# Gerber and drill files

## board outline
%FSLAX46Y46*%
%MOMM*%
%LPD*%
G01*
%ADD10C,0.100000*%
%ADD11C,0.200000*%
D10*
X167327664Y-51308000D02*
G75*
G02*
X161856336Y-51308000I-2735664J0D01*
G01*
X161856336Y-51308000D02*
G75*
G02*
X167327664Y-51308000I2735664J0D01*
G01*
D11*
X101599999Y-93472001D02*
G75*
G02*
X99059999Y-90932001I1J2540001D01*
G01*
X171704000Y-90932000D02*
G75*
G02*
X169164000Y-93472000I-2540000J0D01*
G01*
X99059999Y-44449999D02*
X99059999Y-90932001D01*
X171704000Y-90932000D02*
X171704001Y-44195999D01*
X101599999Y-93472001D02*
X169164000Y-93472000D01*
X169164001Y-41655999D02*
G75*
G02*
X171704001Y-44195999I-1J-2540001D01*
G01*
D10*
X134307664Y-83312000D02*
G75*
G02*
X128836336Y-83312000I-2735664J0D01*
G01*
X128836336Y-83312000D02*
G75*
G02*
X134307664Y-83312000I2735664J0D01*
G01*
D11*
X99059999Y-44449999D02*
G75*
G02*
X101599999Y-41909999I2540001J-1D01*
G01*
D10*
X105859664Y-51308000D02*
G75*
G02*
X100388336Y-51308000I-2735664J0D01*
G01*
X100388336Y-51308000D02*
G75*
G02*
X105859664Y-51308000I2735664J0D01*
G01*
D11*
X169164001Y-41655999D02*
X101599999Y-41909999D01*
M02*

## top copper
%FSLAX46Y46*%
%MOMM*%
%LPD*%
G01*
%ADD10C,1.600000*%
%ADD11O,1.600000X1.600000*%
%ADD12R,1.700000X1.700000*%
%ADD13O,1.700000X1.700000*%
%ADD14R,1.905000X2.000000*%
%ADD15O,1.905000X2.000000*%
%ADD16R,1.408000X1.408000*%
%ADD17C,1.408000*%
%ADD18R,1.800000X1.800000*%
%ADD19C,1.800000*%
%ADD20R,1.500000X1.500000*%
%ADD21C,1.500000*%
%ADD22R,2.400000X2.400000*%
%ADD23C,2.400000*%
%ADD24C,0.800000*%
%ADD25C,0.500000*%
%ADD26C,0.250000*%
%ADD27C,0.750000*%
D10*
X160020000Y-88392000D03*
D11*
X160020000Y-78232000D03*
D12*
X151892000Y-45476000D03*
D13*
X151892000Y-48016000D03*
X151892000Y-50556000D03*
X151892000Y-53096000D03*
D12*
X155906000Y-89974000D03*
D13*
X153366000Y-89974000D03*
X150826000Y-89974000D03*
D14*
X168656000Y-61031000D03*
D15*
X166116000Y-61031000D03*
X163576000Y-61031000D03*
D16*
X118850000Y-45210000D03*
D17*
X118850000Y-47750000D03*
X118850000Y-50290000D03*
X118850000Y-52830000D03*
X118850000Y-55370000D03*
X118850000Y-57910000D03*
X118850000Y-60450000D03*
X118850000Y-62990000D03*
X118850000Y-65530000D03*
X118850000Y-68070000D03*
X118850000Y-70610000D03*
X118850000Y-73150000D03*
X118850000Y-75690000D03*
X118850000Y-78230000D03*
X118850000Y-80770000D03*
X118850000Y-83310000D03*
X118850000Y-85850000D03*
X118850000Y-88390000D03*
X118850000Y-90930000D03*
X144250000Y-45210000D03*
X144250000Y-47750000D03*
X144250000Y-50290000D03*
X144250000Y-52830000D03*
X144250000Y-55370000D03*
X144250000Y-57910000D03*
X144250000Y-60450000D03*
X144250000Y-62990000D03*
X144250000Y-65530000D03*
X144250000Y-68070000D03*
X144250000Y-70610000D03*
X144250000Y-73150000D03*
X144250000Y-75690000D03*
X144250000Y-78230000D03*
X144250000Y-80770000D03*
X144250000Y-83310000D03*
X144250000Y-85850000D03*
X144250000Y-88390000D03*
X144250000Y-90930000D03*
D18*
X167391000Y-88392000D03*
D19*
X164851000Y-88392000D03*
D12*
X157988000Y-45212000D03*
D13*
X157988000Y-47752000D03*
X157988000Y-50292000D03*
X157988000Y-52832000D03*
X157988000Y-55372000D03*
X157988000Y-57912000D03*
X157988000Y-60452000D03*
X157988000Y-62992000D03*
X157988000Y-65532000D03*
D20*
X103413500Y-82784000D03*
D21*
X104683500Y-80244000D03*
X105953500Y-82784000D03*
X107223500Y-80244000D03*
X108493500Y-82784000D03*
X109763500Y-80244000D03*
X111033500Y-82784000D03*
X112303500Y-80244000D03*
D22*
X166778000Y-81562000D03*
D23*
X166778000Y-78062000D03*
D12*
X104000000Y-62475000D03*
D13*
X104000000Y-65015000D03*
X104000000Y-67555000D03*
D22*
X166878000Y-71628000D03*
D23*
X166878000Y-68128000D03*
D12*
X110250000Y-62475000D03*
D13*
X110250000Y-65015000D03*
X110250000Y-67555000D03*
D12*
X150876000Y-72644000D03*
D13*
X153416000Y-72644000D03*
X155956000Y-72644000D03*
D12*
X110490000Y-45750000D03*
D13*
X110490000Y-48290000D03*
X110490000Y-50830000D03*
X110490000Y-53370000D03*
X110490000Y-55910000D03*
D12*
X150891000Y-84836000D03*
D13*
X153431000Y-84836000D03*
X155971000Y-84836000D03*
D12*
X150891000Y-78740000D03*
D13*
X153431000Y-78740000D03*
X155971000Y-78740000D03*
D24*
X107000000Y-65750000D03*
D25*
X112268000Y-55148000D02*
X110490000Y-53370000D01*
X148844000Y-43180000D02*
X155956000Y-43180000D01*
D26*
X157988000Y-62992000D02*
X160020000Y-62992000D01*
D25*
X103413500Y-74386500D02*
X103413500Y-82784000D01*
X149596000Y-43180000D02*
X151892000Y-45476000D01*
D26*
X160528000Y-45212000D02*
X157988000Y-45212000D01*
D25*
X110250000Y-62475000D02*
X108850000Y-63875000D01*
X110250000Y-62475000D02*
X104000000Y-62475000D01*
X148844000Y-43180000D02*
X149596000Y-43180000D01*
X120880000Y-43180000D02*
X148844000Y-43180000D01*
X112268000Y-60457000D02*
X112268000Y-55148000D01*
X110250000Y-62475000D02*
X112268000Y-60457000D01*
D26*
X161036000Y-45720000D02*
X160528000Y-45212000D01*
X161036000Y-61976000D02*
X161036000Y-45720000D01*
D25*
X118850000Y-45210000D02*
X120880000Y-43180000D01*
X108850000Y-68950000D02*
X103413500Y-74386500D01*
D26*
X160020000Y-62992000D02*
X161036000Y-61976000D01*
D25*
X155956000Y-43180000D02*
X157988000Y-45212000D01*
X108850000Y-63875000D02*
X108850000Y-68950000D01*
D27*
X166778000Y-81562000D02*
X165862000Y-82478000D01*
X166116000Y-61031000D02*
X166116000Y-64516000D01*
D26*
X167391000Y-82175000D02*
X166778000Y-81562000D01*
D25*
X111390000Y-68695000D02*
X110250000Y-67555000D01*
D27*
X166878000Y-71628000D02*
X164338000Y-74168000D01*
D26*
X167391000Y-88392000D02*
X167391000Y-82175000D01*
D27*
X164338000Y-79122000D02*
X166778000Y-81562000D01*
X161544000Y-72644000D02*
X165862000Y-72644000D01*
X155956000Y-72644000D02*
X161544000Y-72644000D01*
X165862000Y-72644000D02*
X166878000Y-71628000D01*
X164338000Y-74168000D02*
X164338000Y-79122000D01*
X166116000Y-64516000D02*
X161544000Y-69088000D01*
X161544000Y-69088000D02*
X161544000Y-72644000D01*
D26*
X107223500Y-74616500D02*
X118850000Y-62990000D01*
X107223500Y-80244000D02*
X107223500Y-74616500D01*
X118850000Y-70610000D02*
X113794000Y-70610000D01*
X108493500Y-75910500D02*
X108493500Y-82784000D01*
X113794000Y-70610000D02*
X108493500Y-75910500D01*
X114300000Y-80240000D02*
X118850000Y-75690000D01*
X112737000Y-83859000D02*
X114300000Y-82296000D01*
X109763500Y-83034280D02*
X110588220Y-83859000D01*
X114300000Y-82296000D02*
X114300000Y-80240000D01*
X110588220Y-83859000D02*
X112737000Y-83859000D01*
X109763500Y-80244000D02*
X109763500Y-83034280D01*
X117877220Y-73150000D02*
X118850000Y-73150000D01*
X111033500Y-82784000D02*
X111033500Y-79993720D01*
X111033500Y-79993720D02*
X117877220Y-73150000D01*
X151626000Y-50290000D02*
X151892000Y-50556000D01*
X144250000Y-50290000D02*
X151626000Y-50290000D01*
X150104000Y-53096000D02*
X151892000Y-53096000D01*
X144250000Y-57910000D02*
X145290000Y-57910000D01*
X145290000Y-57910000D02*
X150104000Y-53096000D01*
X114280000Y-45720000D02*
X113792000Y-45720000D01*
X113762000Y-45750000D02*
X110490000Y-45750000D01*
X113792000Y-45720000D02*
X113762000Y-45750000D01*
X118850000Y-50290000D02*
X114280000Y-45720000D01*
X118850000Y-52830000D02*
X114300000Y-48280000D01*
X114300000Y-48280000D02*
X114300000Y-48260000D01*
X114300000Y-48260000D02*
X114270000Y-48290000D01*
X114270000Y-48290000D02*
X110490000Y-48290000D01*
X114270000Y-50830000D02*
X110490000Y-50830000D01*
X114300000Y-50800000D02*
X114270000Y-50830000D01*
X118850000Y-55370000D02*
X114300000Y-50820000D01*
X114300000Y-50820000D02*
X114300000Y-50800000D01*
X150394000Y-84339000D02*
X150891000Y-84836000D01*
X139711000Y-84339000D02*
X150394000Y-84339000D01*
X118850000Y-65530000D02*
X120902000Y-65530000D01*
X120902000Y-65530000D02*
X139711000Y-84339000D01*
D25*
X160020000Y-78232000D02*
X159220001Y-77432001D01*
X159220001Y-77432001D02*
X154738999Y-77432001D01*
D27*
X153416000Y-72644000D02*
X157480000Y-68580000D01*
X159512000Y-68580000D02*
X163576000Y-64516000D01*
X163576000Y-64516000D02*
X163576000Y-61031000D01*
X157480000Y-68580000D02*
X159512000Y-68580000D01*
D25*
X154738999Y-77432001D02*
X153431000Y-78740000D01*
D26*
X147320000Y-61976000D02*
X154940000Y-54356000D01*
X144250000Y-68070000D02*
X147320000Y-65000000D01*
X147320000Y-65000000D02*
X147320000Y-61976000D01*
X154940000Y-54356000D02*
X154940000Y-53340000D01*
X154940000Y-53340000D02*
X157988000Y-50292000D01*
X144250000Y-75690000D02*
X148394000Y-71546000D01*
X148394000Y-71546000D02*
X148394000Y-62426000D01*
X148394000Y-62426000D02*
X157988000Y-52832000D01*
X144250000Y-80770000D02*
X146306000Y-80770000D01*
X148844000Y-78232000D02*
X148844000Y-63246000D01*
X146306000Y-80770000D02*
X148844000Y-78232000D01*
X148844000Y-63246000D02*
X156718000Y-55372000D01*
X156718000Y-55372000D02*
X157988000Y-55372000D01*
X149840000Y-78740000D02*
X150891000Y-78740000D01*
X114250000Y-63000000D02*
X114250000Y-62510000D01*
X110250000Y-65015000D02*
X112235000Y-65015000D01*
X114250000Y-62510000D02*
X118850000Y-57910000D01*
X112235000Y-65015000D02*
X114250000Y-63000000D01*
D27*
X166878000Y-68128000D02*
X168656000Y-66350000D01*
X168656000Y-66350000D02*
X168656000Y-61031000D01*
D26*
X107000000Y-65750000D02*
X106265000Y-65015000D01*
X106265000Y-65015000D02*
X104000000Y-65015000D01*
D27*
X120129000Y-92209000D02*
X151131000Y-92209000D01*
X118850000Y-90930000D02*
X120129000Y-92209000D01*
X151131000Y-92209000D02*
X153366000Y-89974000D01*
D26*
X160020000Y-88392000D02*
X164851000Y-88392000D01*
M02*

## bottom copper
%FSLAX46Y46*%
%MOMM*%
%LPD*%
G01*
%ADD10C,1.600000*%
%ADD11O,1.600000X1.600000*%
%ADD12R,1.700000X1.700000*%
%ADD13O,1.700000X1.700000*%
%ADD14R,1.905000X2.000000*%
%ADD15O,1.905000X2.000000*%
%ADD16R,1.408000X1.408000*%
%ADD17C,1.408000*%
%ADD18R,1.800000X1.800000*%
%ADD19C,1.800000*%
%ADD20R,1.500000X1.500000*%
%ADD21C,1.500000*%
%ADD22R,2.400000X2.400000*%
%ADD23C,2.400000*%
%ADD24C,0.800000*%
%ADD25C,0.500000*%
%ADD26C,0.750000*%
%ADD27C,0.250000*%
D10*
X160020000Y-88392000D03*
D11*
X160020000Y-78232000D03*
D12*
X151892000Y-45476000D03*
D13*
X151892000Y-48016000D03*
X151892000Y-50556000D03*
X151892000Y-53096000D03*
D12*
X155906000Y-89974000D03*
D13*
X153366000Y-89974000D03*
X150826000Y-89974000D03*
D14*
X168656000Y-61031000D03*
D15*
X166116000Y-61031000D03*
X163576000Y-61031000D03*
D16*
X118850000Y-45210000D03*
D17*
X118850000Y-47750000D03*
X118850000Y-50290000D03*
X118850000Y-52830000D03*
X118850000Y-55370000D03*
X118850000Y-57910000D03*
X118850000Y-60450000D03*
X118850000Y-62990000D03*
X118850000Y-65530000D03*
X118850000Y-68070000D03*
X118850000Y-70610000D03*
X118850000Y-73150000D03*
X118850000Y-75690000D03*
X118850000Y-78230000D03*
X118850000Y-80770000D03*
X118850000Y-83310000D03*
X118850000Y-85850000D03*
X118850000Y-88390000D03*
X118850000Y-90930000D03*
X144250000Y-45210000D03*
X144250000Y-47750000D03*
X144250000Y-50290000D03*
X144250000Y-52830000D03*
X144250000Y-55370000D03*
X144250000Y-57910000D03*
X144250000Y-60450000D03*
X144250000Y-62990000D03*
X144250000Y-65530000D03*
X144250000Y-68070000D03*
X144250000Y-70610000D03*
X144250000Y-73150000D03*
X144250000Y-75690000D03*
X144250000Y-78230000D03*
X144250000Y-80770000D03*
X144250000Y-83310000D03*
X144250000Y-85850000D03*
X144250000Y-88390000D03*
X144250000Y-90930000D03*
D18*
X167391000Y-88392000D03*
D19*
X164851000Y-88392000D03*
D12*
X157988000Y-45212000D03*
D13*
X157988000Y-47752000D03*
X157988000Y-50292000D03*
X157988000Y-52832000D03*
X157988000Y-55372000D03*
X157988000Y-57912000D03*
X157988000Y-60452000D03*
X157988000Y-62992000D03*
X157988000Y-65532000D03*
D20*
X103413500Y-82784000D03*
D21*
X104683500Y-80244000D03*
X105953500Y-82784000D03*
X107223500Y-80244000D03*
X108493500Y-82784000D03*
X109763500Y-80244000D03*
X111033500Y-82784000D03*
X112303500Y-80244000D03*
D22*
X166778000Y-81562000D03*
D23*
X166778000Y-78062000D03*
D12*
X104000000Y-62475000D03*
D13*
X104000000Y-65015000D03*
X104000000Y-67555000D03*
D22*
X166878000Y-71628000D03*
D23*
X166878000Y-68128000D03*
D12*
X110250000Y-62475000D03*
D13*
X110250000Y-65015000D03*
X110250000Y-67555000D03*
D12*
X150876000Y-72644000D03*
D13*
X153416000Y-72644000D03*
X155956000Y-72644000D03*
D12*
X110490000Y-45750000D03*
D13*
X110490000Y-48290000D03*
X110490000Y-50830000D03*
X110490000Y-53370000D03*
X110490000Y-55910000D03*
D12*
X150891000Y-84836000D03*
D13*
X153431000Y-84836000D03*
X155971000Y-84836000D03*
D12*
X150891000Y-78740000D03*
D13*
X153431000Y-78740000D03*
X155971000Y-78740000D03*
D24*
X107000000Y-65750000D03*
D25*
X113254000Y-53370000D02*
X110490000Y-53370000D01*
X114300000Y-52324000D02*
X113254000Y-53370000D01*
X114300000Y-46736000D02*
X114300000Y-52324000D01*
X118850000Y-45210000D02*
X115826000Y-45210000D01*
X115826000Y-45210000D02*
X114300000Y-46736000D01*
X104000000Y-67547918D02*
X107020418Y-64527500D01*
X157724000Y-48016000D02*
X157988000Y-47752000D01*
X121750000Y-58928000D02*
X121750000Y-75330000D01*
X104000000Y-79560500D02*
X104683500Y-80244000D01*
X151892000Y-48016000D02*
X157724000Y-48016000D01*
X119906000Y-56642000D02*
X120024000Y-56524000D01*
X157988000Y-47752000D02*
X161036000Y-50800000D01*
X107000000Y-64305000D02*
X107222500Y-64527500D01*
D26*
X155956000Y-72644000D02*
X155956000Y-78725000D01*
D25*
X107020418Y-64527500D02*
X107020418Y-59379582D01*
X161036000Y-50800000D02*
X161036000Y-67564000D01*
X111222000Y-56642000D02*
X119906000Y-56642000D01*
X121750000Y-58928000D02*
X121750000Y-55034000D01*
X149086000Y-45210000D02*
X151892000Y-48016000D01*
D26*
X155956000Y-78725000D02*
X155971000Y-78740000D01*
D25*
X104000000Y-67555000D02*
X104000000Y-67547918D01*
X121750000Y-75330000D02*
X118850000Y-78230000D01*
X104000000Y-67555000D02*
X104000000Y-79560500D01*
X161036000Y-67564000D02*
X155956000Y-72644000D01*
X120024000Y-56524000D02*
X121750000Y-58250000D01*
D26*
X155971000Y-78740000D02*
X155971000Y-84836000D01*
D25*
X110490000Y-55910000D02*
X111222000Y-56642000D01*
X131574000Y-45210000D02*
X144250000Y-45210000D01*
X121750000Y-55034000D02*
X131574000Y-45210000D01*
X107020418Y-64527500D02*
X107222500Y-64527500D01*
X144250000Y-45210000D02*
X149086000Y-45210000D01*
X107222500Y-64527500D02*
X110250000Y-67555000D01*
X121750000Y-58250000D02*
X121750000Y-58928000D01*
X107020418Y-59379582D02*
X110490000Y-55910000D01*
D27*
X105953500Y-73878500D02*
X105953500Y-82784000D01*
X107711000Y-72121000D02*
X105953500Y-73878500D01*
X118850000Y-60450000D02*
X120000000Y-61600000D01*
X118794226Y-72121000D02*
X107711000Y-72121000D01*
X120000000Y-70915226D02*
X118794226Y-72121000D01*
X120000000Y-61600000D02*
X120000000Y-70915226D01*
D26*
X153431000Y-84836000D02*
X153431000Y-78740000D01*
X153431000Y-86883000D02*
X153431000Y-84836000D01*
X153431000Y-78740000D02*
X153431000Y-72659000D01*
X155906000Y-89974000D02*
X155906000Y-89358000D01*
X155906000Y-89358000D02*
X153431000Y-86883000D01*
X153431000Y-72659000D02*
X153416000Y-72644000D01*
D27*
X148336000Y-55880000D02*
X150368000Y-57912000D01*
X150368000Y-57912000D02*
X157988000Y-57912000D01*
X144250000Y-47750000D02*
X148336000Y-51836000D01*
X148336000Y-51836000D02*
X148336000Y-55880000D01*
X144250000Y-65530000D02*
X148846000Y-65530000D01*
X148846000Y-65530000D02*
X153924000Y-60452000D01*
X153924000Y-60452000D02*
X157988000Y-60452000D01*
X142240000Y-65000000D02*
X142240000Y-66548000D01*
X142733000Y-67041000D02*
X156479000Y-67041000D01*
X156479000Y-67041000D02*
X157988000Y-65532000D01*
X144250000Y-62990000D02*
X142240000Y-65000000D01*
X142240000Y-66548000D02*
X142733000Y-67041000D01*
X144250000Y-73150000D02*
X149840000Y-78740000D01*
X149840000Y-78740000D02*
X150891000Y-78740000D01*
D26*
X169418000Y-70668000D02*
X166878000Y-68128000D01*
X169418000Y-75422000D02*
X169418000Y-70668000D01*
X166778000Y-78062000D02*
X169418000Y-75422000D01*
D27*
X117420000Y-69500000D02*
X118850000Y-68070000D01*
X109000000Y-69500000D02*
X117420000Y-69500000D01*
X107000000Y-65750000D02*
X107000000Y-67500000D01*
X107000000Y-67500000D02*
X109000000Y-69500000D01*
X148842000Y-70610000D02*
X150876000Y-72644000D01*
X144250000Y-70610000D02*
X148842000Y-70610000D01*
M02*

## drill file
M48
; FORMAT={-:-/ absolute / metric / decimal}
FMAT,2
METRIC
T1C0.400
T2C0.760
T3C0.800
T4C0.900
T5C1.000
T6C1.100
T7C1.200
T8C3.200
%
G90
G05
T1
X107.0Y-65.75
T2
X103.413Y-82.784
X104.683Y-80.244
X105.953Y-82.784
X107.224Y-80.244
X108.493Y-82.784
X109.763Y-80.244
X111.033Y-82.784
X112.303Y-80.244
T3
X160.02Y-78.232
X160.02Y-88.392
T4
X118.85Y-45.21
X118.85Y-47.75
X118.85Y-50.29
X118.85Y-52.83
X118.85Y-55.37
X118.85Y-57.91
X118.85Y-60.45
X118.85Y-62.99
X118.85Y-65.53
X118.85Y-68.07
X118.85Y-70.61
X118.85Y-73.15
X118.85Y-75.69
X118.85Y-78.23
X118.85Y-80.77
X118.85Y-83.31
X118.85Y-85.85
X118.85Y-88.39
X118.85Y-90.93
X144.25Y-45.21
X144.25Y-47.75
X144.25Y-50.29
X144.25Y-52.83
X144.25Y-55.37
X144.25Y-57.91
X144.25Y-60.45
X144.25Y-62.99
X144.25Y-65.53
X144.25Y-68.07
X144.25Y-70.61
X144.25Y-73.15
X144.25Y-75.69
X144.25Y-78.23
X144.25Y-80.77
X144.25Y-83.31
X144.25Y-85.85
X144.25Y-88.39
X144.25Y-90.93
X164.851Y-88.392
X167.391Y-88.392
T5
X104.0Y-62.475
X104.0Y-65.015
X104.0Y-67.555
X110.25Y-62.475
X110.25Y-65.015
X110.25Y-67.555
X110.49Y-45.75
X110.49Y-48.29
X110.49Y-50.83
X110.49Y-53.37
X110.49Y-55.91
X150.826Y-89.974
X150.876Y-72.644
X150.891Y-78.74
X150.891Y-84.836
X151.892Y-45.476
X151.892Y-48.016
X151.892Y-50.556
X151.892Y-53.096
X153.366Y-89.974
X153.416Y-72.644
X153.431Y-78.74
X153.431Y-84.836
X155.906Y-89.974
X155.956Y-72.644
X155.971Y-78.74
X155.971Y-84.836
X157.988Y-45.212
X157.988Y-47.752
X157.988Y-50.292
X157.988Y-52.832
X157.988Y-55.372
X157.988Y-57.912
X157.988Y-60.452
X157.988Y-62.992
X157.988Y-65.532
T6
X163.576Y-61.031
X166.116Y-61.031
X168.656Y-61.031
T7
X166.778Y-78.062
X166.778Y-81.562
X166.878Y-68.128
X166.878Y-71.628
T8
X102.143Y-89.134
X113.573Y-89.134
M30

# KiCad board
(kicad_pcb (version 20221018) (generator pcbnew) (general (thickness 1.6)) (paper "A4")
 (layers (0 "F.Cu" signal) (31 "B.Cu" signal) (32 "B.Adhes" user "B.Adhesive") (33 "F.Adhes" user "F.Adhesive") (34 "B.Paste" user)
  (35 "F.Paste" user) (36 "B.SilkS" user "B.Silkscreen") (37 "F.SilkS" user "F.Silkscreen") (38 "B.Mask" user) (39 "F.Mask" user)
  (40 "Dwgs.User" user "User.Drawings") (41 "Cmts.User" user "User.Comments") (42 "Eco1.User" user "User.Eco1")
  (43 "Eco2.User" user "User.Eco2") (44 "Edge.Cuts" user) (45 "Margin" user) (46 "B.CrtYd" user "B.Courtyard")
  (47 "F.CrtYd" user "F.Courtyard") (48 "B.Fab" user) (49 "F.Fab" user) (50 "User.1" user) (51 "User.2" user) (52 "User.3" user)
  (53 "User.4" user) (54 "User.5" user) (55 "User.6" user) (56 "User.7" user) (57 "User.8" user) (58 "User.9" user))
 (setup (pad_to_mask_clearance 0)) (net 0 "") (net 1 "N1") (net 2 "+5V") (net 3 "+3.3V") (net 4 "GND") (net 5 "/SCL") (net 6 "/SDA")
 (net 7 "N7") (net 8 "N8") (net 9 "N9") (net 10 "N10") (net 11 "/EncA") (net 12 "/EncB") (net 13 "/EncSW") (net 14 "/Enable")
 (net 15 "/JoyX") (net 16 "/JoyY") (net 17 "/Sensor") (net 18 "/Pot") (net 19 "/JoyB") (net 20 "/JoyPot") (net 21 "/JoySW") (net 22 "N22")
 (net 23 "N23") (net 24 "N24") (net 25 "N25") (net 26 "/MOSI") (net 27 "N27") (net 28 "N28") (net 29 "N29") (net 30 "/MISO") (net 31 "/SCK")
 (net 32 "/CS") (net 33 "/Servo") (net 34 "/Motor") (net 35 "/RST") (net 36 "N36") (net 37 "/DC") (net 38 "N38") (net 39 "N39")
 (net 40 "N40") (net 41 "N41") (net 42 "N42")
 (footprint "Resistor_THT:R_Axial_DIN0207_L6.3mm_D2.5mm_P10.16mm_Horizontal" (layer "F.Cu") (at 160.02 88.392 90)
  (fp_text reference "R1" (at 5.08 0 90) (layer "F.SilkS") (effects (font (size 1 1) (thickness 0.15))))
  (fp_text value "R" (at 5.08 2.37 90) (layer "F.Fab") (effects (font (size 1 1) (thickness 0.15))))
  (pad "1" thru_hole circle (at 0 0 90) (size 1.6 1.6) (drill 0.8) (layers "*.Cu" "*.Mask") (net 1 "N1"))
  (pad "2" thru_hole oval (at 10.16 0 90) (size 1.6 1.6) (drill 0.8) (layers "*.Cu" "*.Mask") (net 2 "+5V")))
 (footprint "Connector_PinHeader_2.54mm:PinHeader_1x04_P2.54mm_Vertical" (layer "F.Cu") (at 151.892 45.476)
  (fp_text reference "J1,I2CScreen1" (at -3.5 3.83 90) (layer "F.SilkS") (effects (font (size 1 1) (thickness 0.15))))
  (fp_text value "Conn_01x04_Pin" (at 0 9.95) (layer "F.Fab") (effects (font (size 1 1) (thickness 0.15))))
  (pad "1" thru_hole rect (at 0 0) (size 1.7 1.7) (drill 1) (layers "*.Cu" "*.Mask") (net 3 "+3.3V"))
  (pad "2" thru_hole oval (at 0 2.54) (size 1.7 1.7) (drill 1) (layers "*.Cu" "*.Mask") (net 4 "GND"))
  (pad "3" thru_hole oval (at 0 5.08) (size 1.7 1.7) (drill 1) (layers "*.Cu" "*.Mask") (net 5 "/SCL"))
  (pad "4" thru_hole oval (at 0 7.62) (size 1.7 1.7) (drill 1) (layers "*.Cu" "*.Mask") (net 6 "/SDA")))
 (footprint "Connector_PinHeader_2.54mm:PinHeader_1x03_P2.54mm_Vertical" (layer "F.Cu") (at 155.906 89.974 -90)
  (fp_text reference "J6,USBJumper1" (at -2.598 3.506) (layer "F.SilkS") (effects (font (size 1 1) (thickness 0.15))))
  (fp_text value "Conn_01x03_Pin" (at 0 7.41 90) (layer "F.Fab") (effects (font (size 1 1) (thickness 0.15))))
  (pad "1" thru_hole rect (at 0 0 270) (size 1.7 1.7) (drill 1) (layers "*.Cu" "*.Mask") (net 2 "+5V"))
  (pad "2" thru_hole oval (at 0 2.54 270) (size 1.7 1.7) (drill 1) (layers "*.Cu" "*.Mask") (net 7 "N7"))
  (pad "3" thru_hole oval (at 0 5.08 270) (size 1.7 1.7) (drill 1) (layers "*.Cu" "*.Mask") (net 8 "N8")))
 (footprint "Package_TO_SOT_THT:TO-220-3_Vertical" (layer "F.Cu") (at 168.656 61.031 180)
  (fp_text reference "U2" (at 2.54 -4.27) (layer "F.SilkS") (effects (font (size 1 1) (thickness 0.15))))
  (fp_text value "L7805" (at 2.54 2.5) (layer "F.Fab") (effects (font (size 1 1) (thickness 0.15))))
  (pad "1" thru_hole rect (at 0 0 180) (size 1.905 2) (drill 1.1) (layers "*.Cu" "*.Mask") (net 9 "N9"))
  (pad "2" thru_hole oval (at 2.54 0 180) (size 1.905 2) (drill 1.1) (layers "*.Cu" "*.Mask") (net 4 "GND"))
  (pad "3" thru_hole oval (at 5.08 0 180) (size 1.905 2) (drill 1.1) (layers "*.Cu" "*.Mask") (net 2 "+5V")))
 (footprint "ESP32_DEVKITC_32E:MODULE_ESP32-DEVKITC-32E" (layer "F.Cu") (at 131.55 68.045)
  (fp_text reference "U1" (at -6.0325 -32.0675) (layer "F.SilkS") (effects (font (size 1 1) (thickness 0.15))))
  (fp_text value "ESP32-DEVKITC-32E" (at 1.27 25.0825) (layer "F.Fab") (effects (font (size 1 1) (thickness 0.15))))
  (pad "J2_1" thru_hole rect (at -12.7 -22.835) (size 1.408 1.408) (drill 0.9) (layers "*.Cu" "*.Mask") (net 3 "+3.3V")
   (solder_mask_margin 0.102))
  (pad "J2_2" thru_hole circle (at -12.7 -20.295) (size 1.408 1.408) (drill 0.9) (layers "*.Cu" "*.Mask") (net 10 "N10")
   (solder_mask_margin 0.102))
  (pad "J2_3" thru_hole circle (at -12.7 -17.755) (size 1.408 1.408) (drill 0.9) (layers "*.Cu" "*.Mask") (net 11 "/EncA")
   (solder_mask_margin 0.102))
  (pad "J2_4" thru_hole circle (at -12.7 -15.215) (size 1.408 1.408) (drill 0.9) (layers "*.Cu" "*.Mask") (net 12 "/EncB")
   (solder_mask_margin 0.102))
  (pad "J2_5" thru_hole circle (at -12.7 -12.675) (size 1.408 1.408) (drill 0.9) (layers "*.Cu" "*.Mask") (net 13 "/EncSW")
   (solder_mask_margin 0.102))
  (pad "J2_6" thru_hole circle (at -12.7 -10.135) (size 1.408 1.408) (drill 0.9) (layers "*.Cu" "*.Mask") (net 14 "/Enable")
   (solder_mask_margin 0.102))
  (pad "J2_7" thru_hole circle (at -12.7 -7.595) (size 1.408 1.408) (drill 0.9) (layers "*.Cu" "*.Mask") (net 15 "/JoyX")
   (solder_mask_margin 0.102))
  (pad "J2_8" thru_hole circle (at -12.7 -5.055) (size 1.408 1.408) (drill 0.9) (layers "*.Cu" "*.Mask") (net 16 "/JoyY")
   (solder_mask_margin 0.102))
  (pad "J2_9" thru_hole circle (at -12.7 -2.515) (size 1.408 1.408) (drill 0.9) (layers "*.Cu" "*.Mask") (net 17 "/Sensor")
   (solder_mask_margin 0.102))
  (pad "J2_10" thru_hole circle (at -12.7 0.025) (size 1.408 1.408) (drill 0.9) (layers "*.Cu" "*.Mask") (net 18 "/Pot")
   (solder_mask_margin 0.102))
  (pad "J2_11" thru_hole circle (at -12.7 2.565) (size 1.408 1.408) (drill 0.9) (layers "*.Cu" "*.Mask") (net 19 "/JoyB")
   (solder_mask_margin 0.102))
  (pad "J2_12" thru_hole circle (at -12.7 5.105) (size 1.408 1.408) (drill 0.9) (layers "*.Cu" "*.Mask") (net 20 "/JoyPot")
   (solder_mask_margin 0.102))
  (pad "J2_13" thru_hole circle (at -12.7 7.645) (size 1.408 1.408) (drill 0.9) (layers "*.Cu" "*.Mask") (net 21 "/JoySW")
   (solder_mask_margin 0.102))
  (pad "J2_14" thru_hole circle (at -12.7 10.185) (size 1.408 1.408) (drill 0.9) (layers "*.Cu" "*.Mask") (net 4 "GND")
   (solder_mask_margin 0.102))
  (pad "J2_15" thru_hole circle (at -12.7 12.725) (size 1.408 1.408) (drill 0.9) (layers "*.Cu" "*.Mask") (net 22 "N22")
   (solder_mask_margin 0.102))
  (pad "J2_16" thru_hole circle (at -12.7 15.265) (size 1.408 1.408) (drill 0.9) (layers "*.Cu" "*.Mask") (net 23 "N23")
   (solder_mask_margin 0.102))
  (pad "J2_17" thru_hole circle (at -12.7 17.805) (size 1.408 1.408) (drill 0.9) (layers "*.Cu" "*.Mask") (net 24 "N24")
   (solder_mask_margin 0.102))
  (pad "J2_18" thru_hole circle (at -12.7 20.345) (size 1.408 1.408) (drill 0.9) (layers "*.Cu" "*.Mask") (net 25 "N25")
   (solder_mask_margin 0.102))
  (pad "J2_19" thru_hole circle (at -12.7 22.885) (size 1.408 1.408) (drill 0.9) (layers "*.Cu" "*.Mask") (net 7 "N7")
   (solder_mask_margin 0.102))
  (pad "J3_1" thru_hole circle (at 12.7 -22.835) (size 1.408 1.408) (drill 0.9) (layers "*.Cu" "*.Mask") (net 4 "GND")
   (solder_mask_margin 0.102))
  (pad "J3_2" thru_hole circle (at 12.7 -20.295) (size 1.408 1.408) (drill 0.9) (layers "*.Cu" "*.Mask") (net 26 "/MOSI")
   (solder_mask_margin 0.102))
  (pad "J3_3" thru_hole circle (at 12.7 -17.755) (size 1.408 1.408) (drill 0.9) (layers "*.Cu" "*.Mask") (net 5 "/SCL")
   (solder_mask_margin 0.102))
  (pad "J3_4" thru_hole circle (at 12.7 -15.215) (size 1.408 1.408) (drill 0.9) (layers "*.Cu" "*.Mask") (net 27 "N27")
   (solder_mask_margin 0.102))
  (pad "J3_5" thru_hole circle (at 12.7 -12.675) (size 1.408 1.408) (drill 0.9) (layers "*.Cu" "*.Mask") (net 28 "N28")
   (solder_mask_margin 0.102))
  (pad "J3_6" thru_hole circle (at 12.7 -10.135) (size 1.408 1.408) (drill 0.9) (layers "*.Cu" "*.Mask") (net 6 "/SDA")
   (solder_mask_margin 0.102))
  (pad "J3_7" thru_hole circle (at 12.7 -7.595) (size 1.408 1.408) (drill 0.9) (layers "*.Cu" "*.Mask") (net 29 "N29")
   (solder_mask_margin 0.102))
  (pad "J3_8" thru_hole circle (at 12.7 -5.055) (size 1.408 1.408) (drill 0.9) (layers "*.Cu" "*.Mask") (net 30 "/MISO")
   (solder_mask_margin 0.102))
  (pad "J3_9" thru_hole circle (at 12.7 -2.515) (size 1.408 1.408) (drill 0.9) (layers "*.Cu" "*.Mask") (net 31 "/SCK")
   (solder_mask_margin 0.102))
  (pad "J3_10" thru_hole circle (at 12.7 0.025) (size 1.408 1.408) (drill 0.9) (layers "*.Cu" "*.Mask") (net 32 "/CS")
   (solder_mask_margin 0.102))
  (pad "J3_11" thru_hole circle (at 12.7 2.565) (size 1.408 1.408) (drill 0.9) (layers "*.Cu" "*.Mask") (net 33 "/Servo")
   (solder_mask_margin 0.102))
  (pad "J3_12" thru_hole circle (at 12.7 5.105) (size 1.408 1.408) (drill 0.9) (layers "*.Cu" "*.Mask") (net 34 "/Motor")
   (solder_mask_margin 0.102))
  (pad "J3_13" thru_hole circle (at 12.7 7.645) (size 1.408 1.408) (drill 0.9) (layers "*.Cu" "*.Mask") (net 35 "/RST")
   (solder_mask_margin 0.102))
  (pad "J3_14" thru_hole circle (at 12.7 10.185) (size 1.408 1.408) (drill 0.9) (layers "*.Cu" "*.Mask") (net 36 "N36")
   (solder_mask_margin 0.102))
  (pad "J3_15" thru_hole circle (at 12.7 12.725) (size 1.408 1.408) (drill 0.9) (layers "*.Cu" "*.Mask") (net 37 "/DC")
   (solder_mask_margin 0.102))
  (pad "J3_16" thru_hole circle (at 12.7 15.265) (size 1.408 1.408) (drill 0.9) (layers "*.Cu" "*.Mask") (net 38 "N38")
   (solder_mask_margin 0.102))
  (pad "J3_17" thru_hole circle (at 12.7 17.805) (size 1.408 1.408) (drill 0.9) (layers "*.Cu" "*.Mask") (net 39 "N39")
   (solder_mask_margin 0.102))
  (pad "J3_18" thru_hole circle (at 12.7 20.345) (size 1.408 1.408) (drill 0.9) (layers "*.Cu" "*.Mask") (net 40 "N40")
   (solder_mask_margin 0.102))
  (pad "J3_19" thru_hole circle (at 12.7 22.885) (size 1.408 1.408) (drill 0.9) (layers "*.Cu" "*.Mask") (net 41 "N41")
   (solder_mask_margin 0.102)))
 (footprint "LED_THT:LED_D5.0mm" (layer "F.Cu") (at 167.391 88.392 180)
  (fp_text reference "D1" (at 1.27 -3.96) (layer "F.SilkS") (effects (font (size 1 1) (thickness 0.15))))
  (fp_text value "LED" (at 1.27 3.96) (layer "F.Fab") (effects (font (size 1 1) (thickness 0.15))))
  (pad "1" thru_hole rect (at 0 0 180) (size 1.8 1.8) (drill 0.9) (layers "*.Cu" "*.Mask") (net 4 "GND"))
  (pad "2" thru_hole circle (at 2.54 0 180) (size 1.8 1.8) (drill 0.9) (layers "*.Cu" "*.Mask") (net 1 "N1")))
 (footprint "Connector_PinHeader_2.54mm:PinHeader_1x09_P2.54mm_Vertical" (layer "F.Cu") (at 157.988 45.212)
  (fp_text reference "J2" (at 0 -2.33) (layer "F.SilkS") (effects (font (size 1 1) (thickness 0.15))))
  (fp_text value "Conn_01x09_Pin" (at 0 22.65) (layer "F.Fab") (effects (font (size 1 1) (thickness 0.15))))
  (pad "1" thru_hole rect (at 0 0) (size 1.7 1.7) (drill 1) (layers "*.Cu" "*.Mask") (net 3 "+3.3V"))
  (pad "2" thru_hole oval (at 0 2.54) (size 1.7 1.7) (drill 1) (layers "*.Cu" "*.Mask") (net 4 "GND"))
  (pad "3" thru_hole oval (at 0 5.08) (size 1.7 1.7) (drill 1) (layers "*.Cu" "*.Mask") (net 32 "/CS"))
  (pad "4" thru_hole oval (at 0 7.62) (size 1.7 1.7) (drill 1) (layers "*.Cu" "*.Mask") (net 35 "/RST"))
  (pad "5" thru_hole oval (at 0 10.16) (size 1.7 1.7) (drill 1) (layers "*.Cu" "*.Mask") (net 37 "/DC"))
  (pad "6" thru_hole oval (at 0 12.7) (size 1.7 1.7) (drill 1) (layers "*.Cu" "*.Mask") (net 26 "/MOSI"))
  (pad "7" thru_hole oval (at 0 15.24) (size 1.7 1.7) (drill 1) (layers "*.Cu" "*.Mask") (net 31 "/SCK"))
  (pad "8" thru_hole oval (at 0 17.78) (size 1.7 1.7) (drill 1) (layers "*.Cu" "*.Mask") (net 3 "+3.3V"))
  (pad "9" thru_hole oval (at 0 20.32) (size 1.7 1.7) (drill 1) (layers "*.Cu" "*.Mask") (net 30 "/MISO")))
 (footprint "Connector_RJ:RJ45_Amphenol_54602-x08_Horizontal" (layer "F.Cu") (at 103.4135 82.784)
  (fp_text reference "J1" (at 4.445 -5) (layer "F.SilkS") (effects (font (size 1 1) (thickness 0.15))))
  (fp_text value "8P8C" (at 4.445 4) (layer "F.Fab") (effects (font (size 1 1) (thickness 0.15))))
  (pad "" np_thru_hole circle (at -1.27 6.35) (size 3.2 3.2) (drill 3.2) (layers "*.Cu" "*.Mask"))
  (pad "" np_thru_hole circle (at 10.16 6.35) (size 3.2 3.2) (drill 3.2) (layers "*.Cu" "*.Mask"))
  (pad "1" thru_hole rect (at 0 0) (size 1.5 1.5) (drill 0.76) (layers "*.Cu" "*.Mask") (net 3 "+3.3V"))
  (pad "2" thru_hole circle (at 1.27 -2.54) (size 1.5 1.5) (drill 0.76) (layers "*.Cu" "*.Mask") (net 4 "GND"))
  (pad "3" thru_hole circle (at 2.54 0) (size 1.5 1.5) (drill 0.76) (layers "*.Cu" "*.Mask") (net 15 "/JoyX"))
  (pad "4" thru_hole circle (at 3.81 -2.54) (size 1.5 1.5) (drill 0.76) (layers "*.Cu" "*.Mask") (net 16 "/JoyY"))
  (pad "5" thru_hole circle (at 5.08 0) (size 1.5 1.5) (drill 0.76) (layers "*.Cu" "*.Mask") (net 19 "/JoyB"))
  (pad "6" thru_hole circle (at 6.35 -2.54) (size 1.5 1.5) (drill 0.76) (layers "*.Cu" "*.Mask") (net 21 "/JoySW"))
  (pad "7" thru_hole circle (at 7.62 0) (size 1.5 1.5) (drill 0.76) (layers "*.Cu" "*.Mask") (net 20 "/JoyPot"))
  (pad "8" thru_hole circle (at 8.89 -2.54) (size 1.5 1.5) (drill 0.76) (layers "*.Cu" "*.Mask") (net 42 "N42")))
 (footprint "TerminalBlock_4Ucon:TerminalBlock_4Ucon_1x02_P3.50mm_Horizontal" (layer "F.Cu") (at 166.778 81.562 90)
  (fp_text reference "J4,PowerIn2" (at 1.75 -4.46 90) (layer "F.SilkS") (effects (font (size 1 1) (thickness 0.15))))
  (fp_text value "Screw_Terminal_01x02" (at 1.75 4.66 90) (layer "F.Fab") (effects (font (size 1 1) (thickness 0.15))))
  (pad "1" thru_hole rect (at 0 0 90) (size 2.4 2.4) (drill 1.2) (layers "*.Cu" "*.Mask") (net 4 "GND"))
  (pad "2" thru_hole circle (at 3.5 0 90) (size 2.4 2.4) (drill 1.2) (layers "*.Cu" "*.Mask") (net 9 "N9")))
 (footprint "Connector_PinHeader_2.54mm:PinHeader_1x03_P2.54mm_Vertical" (layer "F.Cu") (at 104 62.475)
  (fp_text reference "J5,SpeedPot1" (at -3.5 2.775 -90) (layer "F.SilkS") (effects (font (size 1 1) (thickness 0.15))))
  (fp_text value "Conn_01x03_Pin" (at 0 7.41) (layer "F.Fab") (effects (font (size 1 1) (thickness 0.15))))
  (pad "1" thru_hole rect (at 0 0) (size 1.7 1.7) (drill 1) (layers "*.Cu" "*.Mask") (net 3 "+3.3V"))
  (pad "2" thru_hole oval (at 0 2.54) (size 1.7 1.7) (drill 1) (layers "*.Cu" "*.Mask") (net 18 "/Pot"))
  (pad "3" thru_hole oval (at 0 5.08) (size 1.7 1.7) (drill 1) (layers "*.Cu" "*.Mask") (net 4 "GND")))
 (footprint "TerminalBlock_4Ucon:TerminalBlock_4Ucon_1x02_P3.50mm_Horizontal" (layer "F.Cu") (at 166.878 71.628 90)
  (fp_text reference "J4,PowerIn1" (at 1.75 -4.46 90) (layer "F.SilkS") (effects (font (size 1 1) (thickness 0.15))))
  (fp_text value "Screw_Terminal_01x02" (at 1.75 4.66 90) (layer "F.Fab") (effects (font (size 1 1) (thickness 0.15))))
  (pad "1" thru_hole rect (at 0 0 90) (size 2.4 2.4) (drill 1.2) (layers "*.Cu" "*.Mask") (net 4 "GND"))
  (pad "2" thru_hole circle (at 3.5 0 90) (size 2.4 2.4) (drill 1.2) (layers "*.Cu" "*.Mask") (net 9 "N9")))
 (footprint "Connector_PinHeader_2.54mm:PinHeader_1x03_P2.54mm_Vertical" (layer "F.Cu") (at 110.25 62.475)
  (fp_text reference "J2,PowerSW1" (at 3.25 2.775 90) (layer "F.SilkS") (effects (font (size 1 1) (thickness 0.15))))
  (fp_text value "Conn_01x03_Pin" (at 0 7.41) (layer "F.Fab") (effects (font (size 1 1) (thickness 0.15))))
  (pad "1" thru_hole rect (at 0 0) (size 1.7 1.7) (drill 1) (layers "*.Cu" "*.Mask") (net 3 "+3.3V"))
  (pad "2" thru_hole oval (at 0 2.54) (size 1.7 1.7) (drill 1) (layers "*.Cu" "*.Mask") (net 14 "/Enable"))
  (pad "3" thru_hole oval (at 0 5.08) (size 1.7 1.7) (drill 1) (layers "*.Cu" "*.Mask") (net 4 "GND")))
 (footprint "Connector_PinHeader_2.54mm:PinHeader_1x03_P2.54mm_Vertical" (layer "F.Cu") (at 150.876 72.644 90)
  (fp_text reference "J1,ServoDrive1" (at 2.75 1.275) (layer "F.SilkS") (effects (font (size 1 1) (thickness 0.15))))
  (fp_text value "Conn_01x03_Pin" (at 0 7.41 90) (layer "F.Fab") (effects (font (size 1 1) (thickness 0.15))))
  (pad "1" thru_hole rect (at 0 0 90) (size 1.7 1.7) (drill 1) (layers "*.Cu" "*.Mask") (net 33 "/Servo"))
  (pad "2" thru_hole oval (at 0 2.54 90) (size 1.7 1.7) (drill 1) (layers "*.Cu" "*.Mask") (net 2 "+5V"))
  (pad "3" thru_hole oval (at 0 5.08 90) (size 1.7 1.7) (drill 1) (layers "*.Cu" "*.Mask") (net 4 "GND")))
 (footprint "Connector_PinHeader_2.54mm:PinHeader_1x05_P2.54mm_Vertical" (layer "F.Cu") (at 110.49 45.75)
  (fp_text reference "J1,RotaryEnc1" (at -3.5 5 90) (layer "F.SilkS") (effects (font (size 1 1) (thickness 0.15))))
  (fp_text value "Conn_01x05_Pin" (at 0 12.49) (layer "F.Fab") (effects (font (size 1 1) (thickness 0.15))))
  (pad "1" thru_hole rect (at 0 0) (size 1.7 1.7) (drill 1) (layers "*.Cu" "*.Mask") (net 11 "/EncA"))
  (pad "2" thru_hole oval (at 0 2.54) (size 1.7 1.7) (drill 1) (layers "*.Cu" "*.Mask") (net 12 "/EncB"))
  (pad "3" thru_hole oval (at 0 5.08) (size 1.7 1.7) (drill 1) (layers "*.Cu" "*.Mask") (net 13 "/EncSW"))
  (pad "4" thru_hole oval (at 0 7.62) (size 1.7 1.7) (drill 1) (layers "*.Cu" "*.Mask") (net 3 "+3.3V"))
  (pad "5" thru_hole oval (at 0 10.16) (size 1.7 1.7) (drill 1) (layers "*.Cu" "*.Mask") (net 4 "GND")))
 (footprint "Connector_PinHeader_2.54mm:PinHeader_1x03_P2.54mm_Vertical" (layer "F.Cu") (at 150.891 84.836 90)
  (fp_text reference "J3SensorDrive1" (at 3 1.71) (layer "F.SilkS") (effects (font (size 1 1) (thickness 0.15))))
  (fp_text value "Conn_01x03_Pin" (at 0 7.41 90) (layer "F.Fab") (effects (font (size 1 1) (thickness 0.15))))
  (pad "1" thru_hole rect (at 0 0 90) (size 1.7 1.7) (drill 1) (layers "*.Cu" "*.Mask") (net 17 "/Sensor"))
  (pad "2" thru_hole oval (at 0 2.54 90) (size 1.7 1.7) (drill 1) (layers "*.Cu" "*.Mask") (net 2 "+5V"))
  (pad "3" thru_hole oval (at 0 5.08 90) (size 1.7 1.7) (drill 1) (layers "*.Cu" "*.Mask") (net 4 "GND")))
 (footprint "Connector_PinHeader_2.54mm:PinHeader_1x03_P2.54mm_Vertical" (layer "F.Cu") (at 150.891 78.74 90)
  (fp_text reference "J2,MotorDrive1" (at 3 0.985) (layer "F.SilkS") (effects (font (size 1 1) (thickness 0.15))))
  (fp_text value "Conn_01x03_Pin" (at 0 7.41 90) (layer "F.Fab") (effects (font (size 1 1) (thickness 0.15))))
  (pad "1" thru_hole rect (at 0 0 90) (size 1.7 1.7) (drill 1) (layers "*.Cu" "*.Mask") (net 34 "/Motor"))
  (pad "2" thru_hole oval (at 0 2.54 90) (size 1.7 1.7) (drill 1) (layers "*.Cu" "*.Mask") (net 2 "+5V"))
  (pad "3" thru_hole oval (at 0 5.08 90) (size 1.7 1.7) (drill 1) (layers "*.Cu" "*.Mask") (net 4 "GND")))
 (gr_circle (center 164.592 51.308) (end 165.608 53.848) (stroke (width 0.1) (type default)) (fill none) (layer "Edge.Cuts"))
 (gr_arc (start 101.599999 93.472001) (mid 99.803948 92.728052) (end 99.059999 90.932001) (stroke (width 0.2) (type default))
  (layer "Edge.Cuts"))
 (gr_arc (start 171.704 90.932) (mid 170.960051 92.728051) (end 169.164 93.472) (stroke (width 0.2) (type default)) (layer "Edge.Cuts"))
 (gr_line (start 99.059999 44.449999) (end 99.059999 90.932001) (stroke (width 0.2) (type default)) (layer "Edge.Cuts"))
 (gr_line (start 171.704 90.932) (end 171.704001 44.195999) (stroke (width 0.2) (type default)) (layer "Edge.Cuts"))
 (gr_line (start 101.599999 93.472001) (end 169.164 93.472) (stroke (width 0.2) (type default)) (layer "Edge.Cuts"))
 (gr_arc (start 169.164001 41.655999) (mid 170.960052 42.399948) (end 171.704001 44.195999) (stroke (width 0.2) (type default))
  (layer "Edge.Cuts"))
 (gr_circle (center 131.572 83.312) (end 132.588 85.852) (stroke (width 0.1) (type default)) (fill none) (layer "Edge.Cuts"))
 (gr_arc (start 99.059999 44.449999) (mid 99.803948 42.653948) (end 101.599999 41.909999) (stroke (width 0.2) (type default))
  (layer "Edge.Cuts"))
 (gr_circle (center 103.124 51.308) (end 104.14 53.848) (stroke (width 0.1) (type default)) (fill none) (layer "Edge.Cuts"))
 (gr_line (start 169.164001 41.655999) (end 101.599999 41.909999) (stroke (width 0.2) (type default)) (layer "Edge.Cuts"))
 (segment (start 112.268 55.148) (end 110.49 53.37) (width 0.5) (layer "F.Cu") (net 3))
 (segment (start 148.844 43.18) (end 155.956 43.18) (width 0.5) (layer "F.Cu") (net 3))
 (segment (start 157.988 62.992) (end 160.02 62.992) (width 0.25) (layer "F.Cu") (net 3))
 (segment (start 103.4135 74.3865) (end 103.4135 82.784) (width 0.5) (layer "F.Cu") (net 3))
 (segment (start 149.596 43.18) (end 151.892 45.476) (width 0.5) (layer "F.Cu") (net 3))
 (segment (start 160.528 45.212) (end 157.988 45.212) (width 0.25) (layer "F.Cu") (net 3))
 (segment (start 110.25 62.475) (end 108.85 63.875) (width 0.5) (layer "F.Cu") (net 3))
 (segment (start 110.25 62.475) (end 104 62.475) (width 0.5) (layer "F.Cu") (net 3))
 (segment (start 148.844 43.18) (end 149.596 43.18) (width 0.5) (layer "F.Cu") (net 3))
 (segment (start 120.88 43.18) (end 148.844 43.18) (width 0.5) (layer "F.Cu") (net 3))
 (segment (start 112.268 60.457) (end 112.268 55.148) (width 0.5) (layer "F.Cu") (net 3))
 (segment (start 110.25 62.475) (end 112.268 60.457) (width 0.5) (layer "F.Cu") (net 3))
 (segment (start 161.036 45.72) (end 160.528 45.212) (width 0.25) (layer "F.Cu") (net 3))
 (segment (start 161.036 61.976) (end 161.036 45.72) (width 0.25) (layer "F.Cu") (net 3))
 (segment (start 118.85 45.21) (end 120.88 43.18) (width 0.5) (layer "F.Cu") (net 3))
 (segment (start 108.85 68.95) (end 103.4135 74.3865) (width 0.5) (layer "F.Cu") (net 3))
 (segment (start 160.02 62.992) (end 161.036 61.976) (width 0.25) (layer "F.Cu") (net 3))
 (segment (start 155.956 43.18) (end 157.988 45.212) (width 0.5) (layer "F.Cu") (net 3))
 (segment (start 108.85 63.875) (end 108.85 68.95) (width 0.5) (layer "F.Cu") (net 3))
 (segment (start 113.254 53.37) (end 110.49 53.37) (width 0.5) (layer "B.Cu") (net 3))
 (segment (start 114.3 52.324) (end 113.254 53.37) (width 0.5) (layer "B.Cu") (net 3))
 (segment (start 114.3 46.736) (end 114.3 52.324) (width 0.5) (layer "B.Cu") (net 3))
 (segment (start 118.85 45.21) (end 115.826 45.21) (width 0.5) (layer "B.Cu") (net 3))
 (segment (start 115.826 45.21) (end 114.3 46.736) (width 0.5) (layer "B.Cu") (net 3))
 (segment (start 166.778 81.562) (end 165.862 82.478) (width 0.75) (layer "F.Cu") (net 4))
 (segment (start 166.116 61.031) (end 166.116 64.516) (width 0.75) (layer "F.Cu") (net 4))
 (segment (start 167.391 82.175) (end 166.778 81.562) (width 0.25) (layer "F.Cu") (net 4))
 (segment (start 111.39 68.695) (end 110.25 67.555) (width 0.5) (layer "F.Cu") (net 4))
 (segment (start 166.878 71.628) (end 164.338 74.168) (width 0.75) (layer "F.Cu") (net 4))
 (segment (start 167.391 88.392) (end 167.391 82.175) (width 0.25) (layer "F.Cu") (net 4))
 (segment (start 164.338 79.122) (end 166.778 81.562) (width 0.75) (layer "F.Cu") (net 4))
 (segment (start 161.544 72.644) (end 165.862 72.644) (width 0.75) (layer "F.Cu") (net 4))
 (segment (start 155.956 72.644) (end 161.544 72.644) (width 0.75) (layer "F.Cu") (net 4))
 (segment (start 165.862 72.644) (end 166.878 71.628) (width 0.75) (layer "F.Cu") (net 4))
 (segment (start 164.338 74.168) (end 164.338 79.122) (width 0.75) (layer "F.Cu") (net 4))
 (segment (start 166.116 64.516) (end 161.544 69.088) (width 0.75) (layer "F.Cu") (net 4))
 (segment (start 161.544 69.088) (end 161.544 72.644) (width 0.75) (layer "F.Cu") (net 4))
 (segment (start 104 67.547918) (end 107.020418 64.5275) (width 0.5) (layer "B.Cu") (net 4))
 (segment (start 157.724 48.016) (end 157.988 47.752) (width 0.5) (layer "B.Cu") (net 4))
 (segment (start 121.75 58.928) (end 121.75 75.33) (width 0.5) (layer "B.Cu") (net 4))
 (segment (start 104 79.5605) (end 104.6835 80.244) (width 0.5) (layer "B.Cu") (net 4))
 (segment (start 151.892 48.016) (end 157.724 48.016) (width 0.5) (layer "B.Cu") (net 4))
 (segment (start 119.906 56.642) (end 120.024 56.524) (width 0.5) (layer "B.Cu") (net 4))
 (segment (start 157.988 47.752) (end 161.036 50.8) (width 0.5) (layer "B.Cu") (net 4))
 (segment (start 107 64.305) (end 107.2225 64.5275) (width 0.5) (layer "B.Cu") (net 4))
 (segment (start 155.956 72.644) (end 155.956 78.725) (width 0.75) (layer "B.Cu") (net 4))
 (segment (start 107.020418 64.5275) (end 107.020418 59.379582) (width 0.5) (layer "B.Cu") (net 4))
 (segment (start 161.036 50.8) (end 161.036 67.564) (width 0.5) (layer "B.Cu") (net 4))
 (segment (start 111.222 56.642) (end 119.906 56.642) (width 0.5) (layer "B.Cu") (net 4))
 (segment (start 121.75 58.928) (end 121.75 55.034) (width 0.5) (layer "B.Cu") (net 4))
 (segment (start 149.086 45.21) (end 151.892 48.016) (width 0.5) (layer "B.Cu") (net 4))
 (segment (start 155.956 78.725) (end 155.971 78.74) (width 0.75) (layer "B.Cu") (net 4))
 (segment (start 104 67.555) (end 104 67.547918) (width 0.5) (layer "B.Cu") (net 4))
 (segment (start 121.75 75.33) (end 118.85 78.23) (width 0.5) (layer "B.Cu") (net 4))
 (segment (start 104 67.555) (end 104 79.5605) (width 0.5) (layer "B.Cu") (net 4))
 (segment (start 161.036 67.564) (end 155.956 72.644) (width 0.5) (layer "B.Cu") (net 4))
 (segment (start 120.024 56.524) (end 121.75 58.25) (width 0.5) (layer "B.Cu") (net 4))
 (segment (start 155.971 78.74) (end 155.971 84.836) (width 0.75) (layer "B.Cu") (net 4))
 (segment (start 110.49 55.91) (end 111.222 56.642) (width 0.5) (layer "B.Cu") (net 4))
 (segment (start 131.574 45.21) (end 144.25 45.21) (width 0.5) (layer "B.Cu") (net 4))
 (segment (start 121.75 55.034) (end 131.574 45.21) (width 0.5) (layer "B.Cu") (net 4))
 (segment (start 107.020418 64.5275) (end 107.2225 64.5275) (width 0.5) (layer "B.Cu") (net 4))
 (segment (start 144.25 45.21) (end 149.086 45.21) (width 0.5) (layer "B.Cu") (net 4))
 (segment (start 107.2225 64.5275) (end 110.25 67.555) (width 0.5) (layer "B.Cu") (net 4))
 (segment (start 121.75 58.25) (end 121.75 58.928) (width 0.5) (layer "B.Cu") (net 4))
 (segment (start 107.020418 59.379582) (end 110.49 55.91) (width 0.5) (layer "B.Cu") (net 4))
 (segment (start 105.9535 73.8785) (end 105.9535 82.784) (width 0.25) (layer "B.Cu") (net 15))
 (segment (start 107.711 72.121) (end 105.9535 73.8785) (width 0.25) (layer "B.Cu") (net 15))
 (segment (start 118.85 60.45) (end 120 61.6) (width 0.25) (layer "B.Cu") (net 15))
 (segment (start 118.794226 72.121) (end 107.711 72.121) (width 0.25) (layer "B.Cu") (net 15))
 (segment (start 120 70.915226) (end 118.794226 72.121) (width 0.25) (layer "B.Cu") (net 15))
 (segment (start 120 61.6) (end 120 70.915226) (width 0.25) (layer "B.Cu") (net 15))
 (segment (start 107.2235 74.6165) (end 118.85 62.99) (width 0.25) (layer "F.Cu") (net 16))
 (segment (start 107.2235 80.244) (end 107.2235 74.6165) (width 0.25) (layer "F.Cu") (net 16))
 (segment (start 118.85 70.61) (end 113.794 70.61) (width 0.25) (layer "F.Cu") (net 19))
 (segment (start 108.4935 75.9105) (end 108.4935 82.784) (width 0.25) (layer "F.Cu") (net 19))
 (segment (start 113.794 70.61) (end 108.4935 75.9105) (width 0.25) (layer "F.Cu") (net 19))
 (segment (start 114.3 80.24) (end 118.85 75.69) (width 0.25) (layer "F.Cu") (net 21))
 (segment (start 112.737 83.859) (end 114.3 82.296) (width 0.25) (layer "F.Cu") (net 21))
 (segment (start 109.7635 83.03428) (end 110.58822 83.859) (width 0.25) (layer "F.Cu") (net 21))
 (segment (start 114.3 82.296) (end 114.3 80.24) (width 0.25) (layer "F.Cu") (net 21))
 (segment (start 110.58822 83.859) (end 112.737 83.859) (width 0.25) (layer "F.Cu") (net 21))
 (segment (start 109.7635 80.244) (end 109.7635 83.03428) (width 0.25) (layer "F.Cu") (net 21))
 (segment (start 117.87722 73.15) (end 118.85 73.15) (width 0.25) (layer "F.Cu") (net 20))
 (segment (start 111.0335 82.784) (end 111.0335 79.99372) (width 0.25) (layer "F.Cu") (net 20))
 (segment (start 111.0335 79.99372) (end 117.87722 73.15) (width 0.25) (layer "F.Cu") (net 20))
 (segment (start 151.626 50.29) (end 151.892 50.556) (width 0.25) (layer "F.Cu") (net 5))
 (segment (start 144.25 50.29) (end 151.626 50.29) (width 0.25) (layer "F.Cu") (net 5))
 (segment (start 150.104 53.096) (end 151.892 53.096) (width 0.25) (layer "F.Cu") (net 6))
 (segment (start 144.25 57.91) (end 145.29 57.91) (width 0.25) (layer "F.Cu") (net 6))
 (segment (start 145.29 57.91) (end 150.104 53.096) (width 0.25) (layer "F.Cu") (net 6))
 (segment (start 114.28 45.72) (end 113.792 45.72) (width 0.25) (layer "F.Cu") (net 11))
 (segment (start 113.762 45.75) (end 110.49 45.75) (width 0.25) (layer "F.Cu") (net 11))
 (segment (start 113.792 45.72) (end 113.762 45.75) (width 0.25) (layer "F.Cu") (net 11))
 (segment (start 118.85 50.29) (end 114.28 45.72) (width 0.25) (layer "F.Cu") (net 11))
 (segment (start 118.85 52.83) (end 114.3 48.28) (width 0.25) (layer "F.Cu") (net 12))
 (segment (start 114.3 48.28) (end 114.3 48.26) (width 0.25) (layer "F.Cu") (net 12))
 (segment (start 114.3 48.26) (end 114.27 48.29) (width 0.25) (layer "F.Cu") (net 12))
 (segment (start 114.27 48.29) (end 110.49 48.29) (width 0.25) (layer "F.Cu") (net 12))
 (segment (start 114.27 50.83) (end 110.49 50.83) (width 0.25) (layer "F.Cu") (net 13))
 (segment (start 114.3 50.8) (end 114.27 50.83) (width 0.25) (layer "F.Cu") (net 13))
 (segment (start 118.85 55.37) (end 114.3 50.82) (width 0.25) (layer "F.Cu") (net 13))
 (segment (start 114.3 50.82) (end 114.3 50.8) (width 0.25) (layer "F.Cu") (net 13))
 (segment (start 150.394 84.339) (end 150.891 84.836) (width 0.25) (layer "F.Cu") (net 17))
 (segment (start 139.711 84.339) (end 150.394 84.339) (width 0.25) (layer "F.Cu") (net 17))
 (segment (start 118.85 65.53) (end 120.902 65.53) (width 0.25) (layer "F.Cu") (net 17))
 (segment (start 120.902 65.53) (end 139.711 84.339) (width 0.25) (layer "F.Cu") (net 17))
 (segment (start 160.02 78.232) (end 159.220001 77.432001) (width 0.5) (layer "F.Cu") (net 2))
 (segment (start 159.220001 77.432001) (end 154.738999 77.432001) (width 0.5) (layer "F.Cu") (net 2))
 (segment (start 153.416 72.644) (end 157.48 68.58) (width 0.75) (layer "F.Cu") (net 2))
 (segment (start 159.512 68.58) (end 163.576 64.516) (width 0.75) (layer "F.Cu") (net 2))
 (segment (start 163.576 64.516) (end 163.576 61.031) (width 0.75) (layer "F.Cu") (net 2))
 (segment (start 157.48 68.58) (end 159.512 68.58) (width 0.75) (layer "F.Cu") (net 2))
 (segment (start 154.738999 77.432001) (end 153.431 78.74) (width 0.5) (layer "F.Cu") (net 2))
 (segment (start 153.431 84.836) (end 153.431 78.74) (width 0.75) (layer "B.Cu") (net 2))
 (segment (start 153.431 86.883) (end 153.431 84.836) (width 0.75) (layer "B.Cu") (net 2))
 (segment (start 153.431 78.74) (end 153.431 72.659) (width 0.75) (layer "B.Cu") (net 2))
 (segment (start 155.906 89.974) (end 155.906 89.358) (width 0.75) (layer "B.Cu") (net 2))
 (segment (start 155.906 89.358) (end 153.431 86.883) (width 0.75) (layer "B.Cu") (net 2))
 (segment (start 153.431 72.659) (end 153.416 72.644) (width 0.75) (layer "B.Cu") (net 2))
 (segment (start 147.32 61.976) (end 154.94 54.356) (width 0.25) (layer "F.Cu") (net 32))
 (segment (start 144.25 68.07) (end 147.32 65) (width 0.25) (layer "F.Cu") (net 32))
 (segment (start 147.32 65) (end 147.32 61.976) (width 0.25) (layer "F.Cu") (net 32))
 (segment (start 154.94 54.356) (end 154.94 53.34) (width 0.25) (layer "F.Cu") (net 32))
 (segment (start 154.94 53.34) (end 157.988 50.292) (width 0.25) (layer "F.Cu") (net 32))
 (segment (start 144.25 75.69) (end 148.394 71.546) (width 0.25) (layer "F.Cu") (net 35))
 (segment (start 148.394 71.546) (end 148.394 62.426) (width 0.25) (layer "F.Cu") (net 35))
 (segment (start 148.394 62.426) (end 157.988 52.832) (width 0.25) (layer "F.Cu") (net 35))
 (segment (start 144.25 80.77) (end 146.306 80.77) (width 0.25) (layer "F.Cu") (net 37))
 (segment (start 148.844 78.232) (end 148.844 63.246) (width 0.25) (layer "F.Cu") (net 37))
 (segment (start 146.306 80.77) (end 148.844 78.232) (width 0.25) (layer "F.Cu") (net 37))
 (segment (start 148.844 63.246) (end 156.718 55.372) (width 0.25) (layer "F.Cu") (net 37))
 (segment (start 156.718 55.372) (end 157.988 55.372) (width 0.25) (layer "F.Cu") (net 37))
 (segment (start 148.336 55.88) (end 150.368 57.912) (width 0.25) (layer "B.Cu") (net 26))
 (segment (start 150.368 57.912) (end 157.988 57.912) (width 0.25) (layer "B.Cu") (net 26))
 (segment (start 144.25 47.75) (end 148.336 51.836) (width 0.25) (layer "B.Cu") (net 26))
 (segment (start 148.336 51.836) (end 148.336 55.88) (width 0.25) (layer "B.Cu") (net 26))
 (segment (start 144.25 65.53) (end 148.846 65.53) (width 0.25) (layer "B.Cu") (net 31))
 (segment (start 148.846 65.53) (end 153.924 60.452) (width 0.25) (layer "B.Cu") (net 31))
 (segment (start 153.924 60.452) (end 157.988 60.452) (width 0.25) (layer "B.Cu") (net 31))
 (segment (start 142.24 65) (end 142.24 66.548) (width 0.25) (layer "B.Cu") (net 30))
 (segment (start 142.733 67.041) (end 156.479 67.041) (width 0.25) (layer "B.Cu") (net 30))
 (segment (start 156.479 67.041) (end 157.988 65.532) (width 0.25) (layer "B.Cu") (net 30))
 (segment (start 144.25 62.99) (end 142.24 65) (width 0.25) (layer "B.Cu") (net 30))
 (segment (start 142.24 66.548) (end 142.733 67.041) (width 0.25) (layer "B.Cu") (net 30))
 (segment (start 149.84 78.74) (end 150.891 78.74) (width 0.25) (layer "F.Cu") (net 34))
 (segment (start 144.25 73.15) (end 149.84 78.74) (width 0.25) (layer "B.Cu") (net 34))
 (segment (start 149.84 78.74) (end 150.891 78.74) (width 0.25) (layer "B.Cu") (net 34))
 (segment (start 114.25 63) (end 114.25 62.51) (width 0.25) (layer "F.Cu") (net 14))
 (segment (start 110.25 65.015) (end 112.235 65.015) (width 0.25) (layer "F.Cu") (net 14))
 (segment (start 114.25 62.51) (end 118.85 57.91) (width 0.25) (layer "F.Cu") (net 14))
 (segment (start 112.235 65.015) (end 114.25 63) (width 0.25) (layer "F.Cu") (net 14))
 (segment (start 166.878 68.128) (end 168.656 66.35) (width 0.75) (layer "F.Cu") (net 9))
 (segment (start 168.656 66.35) (end 168.656 61.031) (width 0.75) (layer "F.Cu") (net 9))
 (segment (start 169.418 70.668) (end 166.878 68.128) (width 0.75) (layer "B.Cu") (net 9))
 (segment (start 169.418 75.422) (end 169.418 70.668) (width 0.75) (layer "B.Cu") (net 9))
 (segment (start 166.778 78.062) (end 169.418 75.422) (width 0.75) (layer "B.Cu") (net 9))
 (segment (start 107 65.75) (end 106.265 65.015) (width 0.25) (layer "F.Cu") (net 18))
 (segment (start 106.265 65.015) (end 104 65.015) (width 0.25) (layer "F.Cu") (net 18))
 (via (at 107 65.75) (size 0.8) (drill 0.4) (layers "F.Cu" "B.Cu") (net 18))
 (segment (start 117.42 69.5) (end 118.85 68.07) (width 0.25) (layer "B.Cu") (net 18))
 (segment (start 109 69.5) (end 117.42 69.5) (width 0.25) (layer "B.Cu") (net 18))
 (segment (start 107 65.75) (end 107 67.5) (width 0.25) (layer "B.Cu") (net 18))
 (segment (start 107 67.5) (end 109 69.5) (width 0.25) (layer "B.Cu") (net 18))
 (segment (start 120.129 92.209) (end 151.131 92.209) (width 0.75) (layer "F.Cu") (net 7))
 (segment (start 118.85 90.93) (end 120.129 92.209) (width 0.75) (layer "F.Cu") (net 7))
 (segment (start 151.131 92.209) (end 153.366 89.974) (width 0.75) (layer "F.Cu") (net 7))
 (segment (start 148.842 70.61) (end 150.876 72.644) (width 0.25) (layer "B.Cu") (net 33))
 (segment (start 144.25 70.61) (end 148.842 70.61) (width 0.25) (layer "B.Cu") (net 33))
 (segment (start 160.02 88.392) (end 164.851 88.392) (width 0.25) (layer "F.Cu") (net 1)))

